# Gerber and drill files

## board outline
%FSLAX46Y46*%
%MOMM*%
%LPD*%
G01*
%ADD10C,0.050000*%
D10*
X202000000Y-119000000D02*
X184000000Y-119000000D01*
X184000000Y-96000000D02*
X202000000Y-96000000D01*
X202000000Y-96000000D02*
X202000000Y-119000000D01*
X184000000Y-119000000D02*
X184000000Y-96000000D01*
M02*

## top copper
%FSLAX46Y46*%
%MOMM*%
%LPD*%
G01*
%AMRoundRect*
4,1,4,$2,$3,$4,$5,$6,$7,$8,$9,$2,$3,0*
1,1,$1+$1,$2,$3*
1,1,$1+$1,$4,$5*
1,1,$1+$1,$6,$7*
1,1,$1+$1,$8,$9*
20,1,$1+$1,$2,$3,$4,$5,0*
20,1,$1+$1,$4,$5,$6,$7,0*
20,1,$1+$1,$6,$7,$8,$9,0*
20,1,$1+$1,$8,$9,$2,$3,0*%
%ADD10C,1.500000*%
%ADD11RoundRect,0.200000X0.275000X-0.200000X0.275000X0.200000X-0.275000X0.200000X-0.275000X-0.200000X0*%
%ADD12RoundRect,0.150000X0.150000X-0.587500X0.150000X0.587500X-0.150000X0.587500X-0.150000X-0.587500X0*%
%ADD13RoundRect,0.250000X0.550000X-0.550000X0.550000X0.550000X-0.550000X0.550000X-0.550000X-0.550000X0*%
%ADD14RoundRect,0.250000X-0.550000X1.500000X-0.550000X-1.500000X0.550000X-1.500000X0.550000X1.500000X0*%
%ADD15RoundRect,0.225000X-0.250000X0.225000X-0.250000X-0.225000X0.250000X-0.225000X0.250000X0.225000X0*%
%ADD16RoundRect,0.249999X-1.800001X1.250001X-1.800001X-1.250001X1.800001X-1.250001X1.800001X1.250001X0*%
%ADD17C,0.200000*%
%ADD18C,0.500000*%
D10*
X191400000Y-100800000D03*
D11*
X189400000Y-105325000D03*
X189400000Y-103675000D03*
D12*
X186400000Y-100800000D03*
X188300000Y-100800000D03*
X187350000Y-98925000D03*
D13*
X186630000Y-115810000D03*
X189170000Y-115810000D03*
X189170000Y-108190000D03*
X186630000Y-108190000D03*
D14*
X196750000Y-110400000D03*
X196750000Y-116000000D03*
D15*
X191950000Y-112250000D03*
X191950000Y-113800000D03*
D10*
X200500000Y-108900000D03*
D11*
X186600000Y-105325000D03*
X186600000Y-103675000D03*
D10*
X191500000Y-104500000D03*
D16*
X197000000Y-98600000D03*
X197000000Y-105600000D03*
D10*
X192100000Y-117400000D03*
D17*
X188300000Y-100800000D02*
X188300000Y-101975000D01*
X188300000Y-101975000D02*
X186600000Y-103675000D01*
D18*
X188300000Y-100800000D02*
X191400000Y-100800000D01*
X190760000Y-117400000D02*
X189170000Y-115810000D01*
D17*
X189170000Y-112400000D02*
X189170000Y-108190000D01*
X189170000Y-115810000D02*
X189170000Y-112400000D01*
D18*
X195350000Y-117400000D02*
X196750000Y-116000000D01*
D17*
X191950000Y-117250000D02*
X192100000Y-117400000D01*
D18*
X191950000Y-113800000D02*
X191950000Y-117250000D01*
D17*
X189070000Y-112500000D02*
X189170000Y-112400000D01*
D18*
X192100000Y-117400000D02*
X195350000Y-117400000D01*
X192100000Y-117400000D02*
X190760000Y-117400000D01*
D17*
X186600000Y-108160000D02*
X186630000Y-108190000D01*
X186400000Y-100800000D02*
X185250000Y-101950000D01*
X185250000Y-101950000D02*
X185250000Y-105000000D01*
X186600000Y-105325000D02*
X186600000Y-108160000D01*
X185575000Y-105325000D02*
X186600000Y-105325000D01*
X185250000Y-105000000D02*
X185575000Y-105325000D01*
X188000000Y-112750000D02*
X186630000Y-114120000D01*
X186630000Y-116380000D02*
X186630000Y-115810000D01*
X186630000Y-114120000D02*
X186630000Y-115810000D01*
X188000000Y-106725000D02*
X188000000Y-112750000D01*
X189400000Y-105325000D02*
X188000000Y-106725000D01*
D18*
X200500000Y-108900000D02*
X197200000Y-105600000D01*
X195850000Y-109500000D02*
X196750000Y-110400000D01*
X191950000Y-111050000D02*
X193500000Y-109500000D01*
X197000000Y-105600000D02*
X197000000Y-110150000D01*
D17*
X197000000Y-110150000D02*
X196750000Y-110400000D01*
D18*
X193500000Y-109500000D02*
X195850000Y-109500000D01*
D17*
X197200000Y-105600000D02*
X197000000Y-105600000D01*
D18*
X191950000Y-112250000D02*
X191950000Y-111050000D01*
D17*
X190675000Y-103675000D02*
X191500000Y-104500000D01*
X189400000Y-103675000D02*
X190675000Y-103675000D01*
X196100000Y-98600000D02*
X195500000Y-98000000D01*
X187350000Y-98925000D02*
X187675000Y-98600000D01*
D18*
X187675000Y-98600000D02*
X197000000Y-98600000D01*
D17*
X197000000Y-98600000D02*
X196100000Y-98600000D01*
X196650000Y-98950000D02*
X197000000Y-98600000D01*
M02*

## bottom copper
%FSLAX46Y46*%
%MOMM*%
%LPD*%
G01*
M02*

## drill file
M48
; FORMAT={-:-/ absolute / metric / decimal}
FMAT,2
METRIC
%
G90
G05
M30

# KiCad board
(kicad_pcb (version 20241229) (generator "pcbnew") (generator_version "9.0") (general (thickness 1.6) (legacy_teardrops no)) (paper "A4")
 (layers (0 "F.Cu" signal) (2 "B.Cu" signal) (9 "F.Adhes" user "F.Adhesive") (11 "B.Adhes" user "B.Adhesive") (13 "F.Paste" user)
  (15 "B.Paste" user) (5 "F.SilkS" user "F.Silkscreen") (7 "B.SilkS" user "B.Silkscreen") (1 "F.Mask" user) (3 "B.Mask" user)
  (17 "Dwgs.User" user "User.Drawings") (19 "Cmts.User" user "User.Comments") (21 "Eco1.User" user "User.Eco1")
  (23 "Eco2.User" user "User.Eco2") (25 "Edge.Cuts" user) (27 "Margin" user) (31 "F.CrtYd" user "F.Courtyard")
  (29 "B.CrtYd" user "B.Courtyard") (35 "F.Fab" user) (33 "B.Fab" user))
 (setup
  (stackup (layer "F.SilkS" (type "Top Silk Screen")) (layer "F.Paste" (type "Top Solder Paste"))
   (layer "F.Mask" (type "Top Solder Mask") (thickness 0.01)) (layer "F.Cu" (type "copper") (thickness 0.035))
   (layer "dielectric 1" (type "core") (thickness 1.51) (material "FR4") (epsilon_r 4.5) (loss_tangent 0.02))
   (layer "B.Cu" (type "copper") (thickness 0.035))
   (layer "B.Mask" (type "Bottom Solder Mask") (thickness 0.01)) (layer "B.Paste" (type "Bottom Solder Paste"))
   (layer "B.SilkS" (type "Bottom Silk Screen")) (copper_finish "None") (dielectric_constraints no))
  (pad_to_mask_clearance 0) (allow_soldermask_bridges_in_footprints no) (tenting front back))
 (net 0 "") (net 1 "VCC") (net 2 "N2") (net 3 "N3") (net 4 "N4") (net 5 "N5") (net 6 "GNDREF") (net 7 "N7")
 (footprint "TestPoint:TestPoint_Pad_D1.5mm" (layer "F.Cu") (at 191.4 100.8 180)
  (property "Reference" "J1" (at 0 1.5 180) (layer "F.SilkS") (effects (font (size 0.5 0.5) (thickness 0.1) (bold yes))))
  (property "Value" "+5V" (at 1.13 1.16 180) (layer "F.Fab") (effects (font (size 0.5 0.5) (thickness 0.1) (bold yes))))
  (pad "1" smd circle (at 0 0 180) (size 1.5 1.5) (layers "F.Cu" "F.Mask") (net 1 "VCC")))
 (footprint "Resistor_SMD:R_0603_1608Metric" (layer "F.Cu") (at 189.4 104.5 90)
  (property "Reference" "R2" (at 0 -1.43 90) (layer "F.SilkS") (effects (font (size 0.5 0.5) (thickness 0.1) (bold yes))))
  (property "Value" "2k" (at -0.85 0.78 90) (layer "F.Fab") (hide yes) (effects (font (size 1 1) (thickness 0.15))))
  (pad "1" smd roundrect (at -0.825 0 90) (size 0.8 0.95) (layers "F.Cu" "F.Mask" "F.Paste") (roundrect_rratio 0.25) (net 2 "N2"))
  (pad "2" smd roundrect (at 0.825 0 90) (size 0.8 0.95) (layers "F.Cu" "F.Mask" "F.Paste") (roundrect_rratio 0.25) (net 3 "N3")))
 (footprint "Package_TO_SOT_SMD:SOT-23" (layer "F.Cu") (at 187.35 99.8625 90)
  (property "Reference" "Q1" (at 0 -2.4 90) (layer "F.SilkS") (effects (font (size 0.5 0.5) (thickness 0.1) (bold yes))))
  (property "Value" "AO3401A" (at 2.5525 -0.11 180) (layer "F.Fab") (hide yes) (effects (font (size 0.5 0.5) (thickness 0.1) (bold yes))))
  (pad "1" smd roundrect (at -0.9375 -0.95 90) (size 1.475 0.6) (layers "F.Cu" "F.Mask" "F.Paste") (roundrect_rratio 0.25) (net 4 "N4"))
  (pad "2" smd roundrect (at -0.9375 0.95 90) (size 1.475 0.6) (layers "F.Cu" "F.Mask" "F.Paste") (roundrect_rratio 0.25) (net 1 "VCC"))
  (pad "3" smd roundrect (at 0.9375 0 90) (size 1.475 0.6) (layers "F.Cu" "F.Mask" "F.Paste") (roundrect_rratio 0.25) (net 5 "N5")))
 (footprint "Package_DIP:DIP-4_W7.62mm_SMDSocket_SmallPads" (layer "F.Cu") (at 187.9 112 90)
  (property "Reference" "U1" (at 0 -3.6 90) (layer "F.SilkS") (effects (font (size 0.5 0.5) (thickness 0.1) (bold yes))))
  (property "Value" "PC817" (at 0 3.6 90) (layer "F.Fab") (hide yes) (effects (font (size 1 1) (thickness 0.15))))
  (pad "1" smd roundrect (at -3.81 -1.27 90) (size 1.6 1.6) (layers "F.Cu" "F.Mask" "F.Paste") (roundrect_rratio 0.15625) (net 2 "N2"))
  (pad "2" smd roundrect (at -3.81 1.27 90) (size 1.6 1.6) (layers "F.Cu" "F.Mask" "F.Paste") (roundrect_rratio 0.15625) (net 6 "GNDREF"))
  (pad "3" smd roundrect (at 3.81 1.27 90) (size 1.6 1.6) (layers "F.Cu" "F.Mask" "F.Paste") (roundrect_rratio 0.15625) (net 6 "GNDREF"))
  (pad "4" smd roundrect (at 3.81 -1.27 90) (size 1.6 1.6) (layers "F.Cu" "F.Mask" "F.Paste") (roundrect_rratio 0.15625) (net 4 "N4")))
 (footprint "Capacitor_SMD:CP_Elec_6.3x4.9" (layer "F.Cu") (at 196.75 113.2 -90)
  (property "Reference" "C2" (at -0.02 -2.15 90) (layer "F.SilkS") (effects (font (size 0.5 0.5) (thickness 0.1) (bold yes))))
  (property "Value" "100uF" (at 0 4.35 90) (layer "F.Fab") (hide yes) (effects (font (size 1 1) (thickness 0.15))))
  (pad "1" smd roundrect (at -2.8 0 270) (size 3.5 1.6) (layers "F.Cu" "F.Mask" "F.Paste") (roundrect_rratio 0.15625) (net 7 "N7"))
  (pad "2" smd roundrect (at 2.8 0 270) (size 3.5 1.6) (layers "F.Cu" "F.Mask" "F.Paste") (roundrect_rratio 0.15625) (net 6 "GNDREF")))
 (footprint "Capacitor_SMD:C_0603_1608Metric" (layer "F.Cu") (at 191.95 113.025 -90)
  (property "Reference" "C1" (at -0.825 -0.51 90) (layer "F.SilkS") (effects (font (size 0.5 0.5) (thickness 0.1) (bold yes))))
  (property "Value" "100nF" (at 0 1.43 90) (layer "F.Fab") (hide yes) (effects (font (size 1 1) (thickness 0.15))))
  (pad "1" smd roundrect (at -0.775 0 270) (size 0.9 0.95) (layers "F.Cu" "F.Mask" "F.Paste") (roundrect_rratio 0.25) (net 7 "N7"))
  (pad "2" smd roundrect (at 0.775 0 270) (size 0.9 0.95) (layers "F.Cu" "F.Mask" "F.Paste") (roundrect_rratio 0.25) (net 6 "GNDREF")))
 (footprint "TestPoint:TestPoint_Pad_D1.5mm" (layer "F.Cu") (at 200.5 108.9)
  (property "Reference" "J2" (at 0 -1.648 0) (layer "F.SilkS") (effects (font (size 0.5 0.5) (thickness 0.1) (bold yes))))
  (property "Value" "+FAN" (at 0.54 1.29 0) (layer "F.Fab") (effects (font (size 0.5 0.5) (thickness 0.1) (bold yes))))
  (pad "1" smd circle (at 0 0) (size 1.5 1.5) (layers "F.Cu" "F.Mask") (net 7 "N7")))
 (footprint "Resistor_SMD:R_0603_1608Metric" (layer "F.Cu") (at 186.6 104.5 90)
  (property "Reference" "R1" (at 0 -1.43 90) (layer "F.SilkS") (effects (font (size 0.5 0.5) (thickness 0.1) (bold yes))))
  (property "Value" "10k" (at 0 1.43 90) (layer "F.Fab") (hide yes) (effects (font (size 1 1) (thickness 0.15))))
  (pad "1" smd roundrect (at -0.825 0 90) (size 0.8 0.95) (layers "F.Cu" "F.Mask" "F.Paste") (roundrect_rratio 0.25) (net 4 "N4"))
  (pad "2" smd roundrect (at 0.825 0 90) (size 0.8 0.95) (layers "F.Cu" "F.Mask" "F.Paste") (roundrect_rratio 0.25) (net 1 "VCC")))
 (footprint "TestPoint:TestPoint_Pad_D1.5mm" (layer "F.Cu") (at 191.5 104.5)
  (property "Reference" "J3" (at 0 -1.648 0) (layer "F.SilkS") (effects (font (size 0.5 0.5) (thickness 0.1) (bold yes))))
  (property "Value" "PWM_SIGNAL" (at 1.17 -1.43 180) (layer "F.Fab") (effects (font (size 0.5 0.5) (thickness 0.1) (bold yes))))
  (pad "1" smd circle (at 0 0) (size 1.5 1.5) (layers "F.Cu" "F.Mask") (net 3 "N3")))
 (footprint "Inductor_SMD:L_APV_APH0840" (layer "F.Cu") (at 197 102.1 -90)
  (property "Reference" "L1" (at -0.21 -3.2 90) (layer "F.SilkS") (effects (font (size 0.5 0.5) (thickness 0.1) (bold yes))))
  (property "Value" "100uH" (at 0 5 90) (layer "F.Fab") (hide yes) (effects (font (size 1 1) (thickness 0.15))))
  (pad "1" smd roundrect (at -3.5 0 270) (size 3 4.1) (layers "F.Cu" "F.Mask" "F.Paste") (roundrect_rratio 0.083333) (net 5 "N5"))
  (pad "2" smd roundrect (at 3.5 0 270) (size 3 4.1) (layers "F.Cu" "F.Mask" "F.Paste") (roundrect_rratio 0.083333) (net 7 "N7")))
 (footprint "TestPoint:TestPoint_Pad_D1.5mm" (layer "F.Cu") (at 192.1 117.4)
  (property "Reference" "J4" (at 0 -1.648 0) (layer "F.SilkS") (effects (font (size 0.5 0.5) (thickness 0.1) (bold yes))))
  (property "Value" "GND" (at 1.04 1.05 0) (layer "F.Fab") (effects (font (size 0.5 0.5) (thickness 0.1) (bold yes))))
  (pad "1" smd circle (at 0 0) (size 1.5 1.5) (layers "F.Cu" "F.Mask") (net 6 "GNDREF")))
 (gr_line (start 202 119) (end 184 119) (stroke (width 0.05) (type default)) (layer "Edge.Cuts"))
 (gr_line (start 184 96) (end 202 96) (stroke (width 0.05) (type solid)) (layer "Edge.Cuts"))
 (gr_line (start 202 96) (end 202 119) (stroke (width 0.05) (type default)) (layer "Edge.Cuts"))
 (gr_line (start 184 119) (end 184 96) (stroke (width 0.05) (type default)) (layer "Edge.Cuts"))
 (segment (start 188.3 100.8) (end 188.3 101.975) (width 0.2) (layer "F.Cu") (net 1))
 (segment (start 188.3 101.975) (end 186.6 103.675) (width 0.2) (layer "F.Cu") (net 1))
 (segment (start 188.3 100.8) (end 191.4 100.8) (width 0.5) (layer "F.Cu") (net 1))
 (segment (start 190.76 117.4) (end 189.17 115.81) (width 0.5) (layer "F.Cu") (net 6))
 (segment (start 189.17 112.4) (end 189.17 108.19) (width 0.2) (layer "F.Cu") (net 6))
 (segment (start 189.17 115.81) (end 189.17 112.4) (width 0.2) (layer "F.Cu") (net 6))
 (segment (start 195.35 117.4) (end 196.75 116) (width 0.5) (layer "F.Cu") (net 6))
 (segment (start 191.95 117.25) (end 192.1 117.4) (width 0.2) (layer "F.Cu") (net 6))
 (segment (start 191.95 113.8) (end 191.95 117.25) (width 0.5) (layer "F.Cu") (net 6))
 (segment (start 189.07 112.5) (end 189.17 112.4) (width 0.2) (layer "F.Cu") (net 6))
 (segment (start 192.1 117.4) (end 195.35 117.4) (width 0.5) (layer "F.Cu") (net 6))
 (segment (start 192.1 117.4) (end 190.76 117.4) (width 0.5) (layer "F.Cu") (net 6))
 (segment (start 186.6 108.16) (end 186.63 108.19) (width 0.2) (layer "F.Cu") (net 4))
 (segment (start 186.4 100.8) (end 185.25 101.95) (width 0.2) (layer "F.Cu") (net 4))
 (segment (start 185.25 101.95) (end 185.25 105) (width 0.2) (layer "F.Cu") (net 4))
 (segment (start 186.6 105.325) (end 186.6 108.16) (width 0.2) (layer "F.Cu") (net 4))
 (segment (start 185.575 105.325) (end 186.6 105.325) (width 0.2) (layer "F.Cu") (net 4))
 (segment (start 185.25 105) (end 185.575 105.325) (width 0.2) (layer "F.Cu") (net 4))
 (segment (start 188 112.75) (end 186.63 114.12) (width 0.2) (layer "F.Cu") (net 2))
 (segment (start 186.63 116.38) (end 186.63 115.81) (width 0.2) (layer "F.Cu") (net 2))
 (segment (start 186.63 114.12) (end 186.63 115.81) (width 0.2) (layer "F.Cu") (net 2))
 (segment (start 188 106.725) (end 188 112.75) (width 0.2) (layer "F.Cu") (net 2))
 (segment (start 189.4 105.325) (end 188 106.725) (width 0.2) (layer "F.Cu") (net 2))
 (segment (start 200.5 108.9) (end 197.2 105.6) (width 0.5) (layer "F.Cu") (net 7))
 (segment (start 195.85 109.5) (end 196.75 110.4) (width 0.5) (layer "F.Cu") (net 7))
 (segment (start 191.95 111.05) (end 193.5 109.5) (width 0.5) (layer "F.Cu") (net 7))
 (segment (start 197 105.6) (end 197 110.15) (width 0.5) (layer "F.Cu") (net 7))
 (segment (start 197 110.15) (end 196.75 110.4) (width 0.2) (layer "F.Cu") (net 7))
 (segment (start 193.5 109.5) (end 195.85 109.5) (width 0.5) (layer "F.Cu") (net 7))
 (segment (start 197.2 105.6) (end 197 105.6) (width 0.2) (layer "F.Cu") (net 7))
 (segment (start 191.95 112.25) (end 191.95 111.05) (width 0.5) (layer "F.Cu") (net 7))
 (segment (start 190.675 103.675) (end 191.5 104.5) (width 0.2) (layer "F.Cu") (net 3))
 (segment (start 189.4 103.675) (end 190.675 103.675) (width 0.2) (layer "F.Cu") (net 3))
 (segment (start 196.1 98.6) (end 195.5 98) (width 0.2) (layer "F.Cu") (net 5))
 (segment (start 187.35 98.925) (end 187.675 98.6) (width 0.2) (layer "F.Cu") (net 5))
 (segment (start 187.675 98.6) (end 197 98.6) (width 0.5) (layer "F.Cu") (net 5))
 (segment (start 197 98.6) (end 196.1 98.6) (width 0.2) (layer "F.Cu") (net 5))
 (segment (start 196.65 98.95) (end 197 98.6) (width 0.2) (layer "F.Cu") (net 5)))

